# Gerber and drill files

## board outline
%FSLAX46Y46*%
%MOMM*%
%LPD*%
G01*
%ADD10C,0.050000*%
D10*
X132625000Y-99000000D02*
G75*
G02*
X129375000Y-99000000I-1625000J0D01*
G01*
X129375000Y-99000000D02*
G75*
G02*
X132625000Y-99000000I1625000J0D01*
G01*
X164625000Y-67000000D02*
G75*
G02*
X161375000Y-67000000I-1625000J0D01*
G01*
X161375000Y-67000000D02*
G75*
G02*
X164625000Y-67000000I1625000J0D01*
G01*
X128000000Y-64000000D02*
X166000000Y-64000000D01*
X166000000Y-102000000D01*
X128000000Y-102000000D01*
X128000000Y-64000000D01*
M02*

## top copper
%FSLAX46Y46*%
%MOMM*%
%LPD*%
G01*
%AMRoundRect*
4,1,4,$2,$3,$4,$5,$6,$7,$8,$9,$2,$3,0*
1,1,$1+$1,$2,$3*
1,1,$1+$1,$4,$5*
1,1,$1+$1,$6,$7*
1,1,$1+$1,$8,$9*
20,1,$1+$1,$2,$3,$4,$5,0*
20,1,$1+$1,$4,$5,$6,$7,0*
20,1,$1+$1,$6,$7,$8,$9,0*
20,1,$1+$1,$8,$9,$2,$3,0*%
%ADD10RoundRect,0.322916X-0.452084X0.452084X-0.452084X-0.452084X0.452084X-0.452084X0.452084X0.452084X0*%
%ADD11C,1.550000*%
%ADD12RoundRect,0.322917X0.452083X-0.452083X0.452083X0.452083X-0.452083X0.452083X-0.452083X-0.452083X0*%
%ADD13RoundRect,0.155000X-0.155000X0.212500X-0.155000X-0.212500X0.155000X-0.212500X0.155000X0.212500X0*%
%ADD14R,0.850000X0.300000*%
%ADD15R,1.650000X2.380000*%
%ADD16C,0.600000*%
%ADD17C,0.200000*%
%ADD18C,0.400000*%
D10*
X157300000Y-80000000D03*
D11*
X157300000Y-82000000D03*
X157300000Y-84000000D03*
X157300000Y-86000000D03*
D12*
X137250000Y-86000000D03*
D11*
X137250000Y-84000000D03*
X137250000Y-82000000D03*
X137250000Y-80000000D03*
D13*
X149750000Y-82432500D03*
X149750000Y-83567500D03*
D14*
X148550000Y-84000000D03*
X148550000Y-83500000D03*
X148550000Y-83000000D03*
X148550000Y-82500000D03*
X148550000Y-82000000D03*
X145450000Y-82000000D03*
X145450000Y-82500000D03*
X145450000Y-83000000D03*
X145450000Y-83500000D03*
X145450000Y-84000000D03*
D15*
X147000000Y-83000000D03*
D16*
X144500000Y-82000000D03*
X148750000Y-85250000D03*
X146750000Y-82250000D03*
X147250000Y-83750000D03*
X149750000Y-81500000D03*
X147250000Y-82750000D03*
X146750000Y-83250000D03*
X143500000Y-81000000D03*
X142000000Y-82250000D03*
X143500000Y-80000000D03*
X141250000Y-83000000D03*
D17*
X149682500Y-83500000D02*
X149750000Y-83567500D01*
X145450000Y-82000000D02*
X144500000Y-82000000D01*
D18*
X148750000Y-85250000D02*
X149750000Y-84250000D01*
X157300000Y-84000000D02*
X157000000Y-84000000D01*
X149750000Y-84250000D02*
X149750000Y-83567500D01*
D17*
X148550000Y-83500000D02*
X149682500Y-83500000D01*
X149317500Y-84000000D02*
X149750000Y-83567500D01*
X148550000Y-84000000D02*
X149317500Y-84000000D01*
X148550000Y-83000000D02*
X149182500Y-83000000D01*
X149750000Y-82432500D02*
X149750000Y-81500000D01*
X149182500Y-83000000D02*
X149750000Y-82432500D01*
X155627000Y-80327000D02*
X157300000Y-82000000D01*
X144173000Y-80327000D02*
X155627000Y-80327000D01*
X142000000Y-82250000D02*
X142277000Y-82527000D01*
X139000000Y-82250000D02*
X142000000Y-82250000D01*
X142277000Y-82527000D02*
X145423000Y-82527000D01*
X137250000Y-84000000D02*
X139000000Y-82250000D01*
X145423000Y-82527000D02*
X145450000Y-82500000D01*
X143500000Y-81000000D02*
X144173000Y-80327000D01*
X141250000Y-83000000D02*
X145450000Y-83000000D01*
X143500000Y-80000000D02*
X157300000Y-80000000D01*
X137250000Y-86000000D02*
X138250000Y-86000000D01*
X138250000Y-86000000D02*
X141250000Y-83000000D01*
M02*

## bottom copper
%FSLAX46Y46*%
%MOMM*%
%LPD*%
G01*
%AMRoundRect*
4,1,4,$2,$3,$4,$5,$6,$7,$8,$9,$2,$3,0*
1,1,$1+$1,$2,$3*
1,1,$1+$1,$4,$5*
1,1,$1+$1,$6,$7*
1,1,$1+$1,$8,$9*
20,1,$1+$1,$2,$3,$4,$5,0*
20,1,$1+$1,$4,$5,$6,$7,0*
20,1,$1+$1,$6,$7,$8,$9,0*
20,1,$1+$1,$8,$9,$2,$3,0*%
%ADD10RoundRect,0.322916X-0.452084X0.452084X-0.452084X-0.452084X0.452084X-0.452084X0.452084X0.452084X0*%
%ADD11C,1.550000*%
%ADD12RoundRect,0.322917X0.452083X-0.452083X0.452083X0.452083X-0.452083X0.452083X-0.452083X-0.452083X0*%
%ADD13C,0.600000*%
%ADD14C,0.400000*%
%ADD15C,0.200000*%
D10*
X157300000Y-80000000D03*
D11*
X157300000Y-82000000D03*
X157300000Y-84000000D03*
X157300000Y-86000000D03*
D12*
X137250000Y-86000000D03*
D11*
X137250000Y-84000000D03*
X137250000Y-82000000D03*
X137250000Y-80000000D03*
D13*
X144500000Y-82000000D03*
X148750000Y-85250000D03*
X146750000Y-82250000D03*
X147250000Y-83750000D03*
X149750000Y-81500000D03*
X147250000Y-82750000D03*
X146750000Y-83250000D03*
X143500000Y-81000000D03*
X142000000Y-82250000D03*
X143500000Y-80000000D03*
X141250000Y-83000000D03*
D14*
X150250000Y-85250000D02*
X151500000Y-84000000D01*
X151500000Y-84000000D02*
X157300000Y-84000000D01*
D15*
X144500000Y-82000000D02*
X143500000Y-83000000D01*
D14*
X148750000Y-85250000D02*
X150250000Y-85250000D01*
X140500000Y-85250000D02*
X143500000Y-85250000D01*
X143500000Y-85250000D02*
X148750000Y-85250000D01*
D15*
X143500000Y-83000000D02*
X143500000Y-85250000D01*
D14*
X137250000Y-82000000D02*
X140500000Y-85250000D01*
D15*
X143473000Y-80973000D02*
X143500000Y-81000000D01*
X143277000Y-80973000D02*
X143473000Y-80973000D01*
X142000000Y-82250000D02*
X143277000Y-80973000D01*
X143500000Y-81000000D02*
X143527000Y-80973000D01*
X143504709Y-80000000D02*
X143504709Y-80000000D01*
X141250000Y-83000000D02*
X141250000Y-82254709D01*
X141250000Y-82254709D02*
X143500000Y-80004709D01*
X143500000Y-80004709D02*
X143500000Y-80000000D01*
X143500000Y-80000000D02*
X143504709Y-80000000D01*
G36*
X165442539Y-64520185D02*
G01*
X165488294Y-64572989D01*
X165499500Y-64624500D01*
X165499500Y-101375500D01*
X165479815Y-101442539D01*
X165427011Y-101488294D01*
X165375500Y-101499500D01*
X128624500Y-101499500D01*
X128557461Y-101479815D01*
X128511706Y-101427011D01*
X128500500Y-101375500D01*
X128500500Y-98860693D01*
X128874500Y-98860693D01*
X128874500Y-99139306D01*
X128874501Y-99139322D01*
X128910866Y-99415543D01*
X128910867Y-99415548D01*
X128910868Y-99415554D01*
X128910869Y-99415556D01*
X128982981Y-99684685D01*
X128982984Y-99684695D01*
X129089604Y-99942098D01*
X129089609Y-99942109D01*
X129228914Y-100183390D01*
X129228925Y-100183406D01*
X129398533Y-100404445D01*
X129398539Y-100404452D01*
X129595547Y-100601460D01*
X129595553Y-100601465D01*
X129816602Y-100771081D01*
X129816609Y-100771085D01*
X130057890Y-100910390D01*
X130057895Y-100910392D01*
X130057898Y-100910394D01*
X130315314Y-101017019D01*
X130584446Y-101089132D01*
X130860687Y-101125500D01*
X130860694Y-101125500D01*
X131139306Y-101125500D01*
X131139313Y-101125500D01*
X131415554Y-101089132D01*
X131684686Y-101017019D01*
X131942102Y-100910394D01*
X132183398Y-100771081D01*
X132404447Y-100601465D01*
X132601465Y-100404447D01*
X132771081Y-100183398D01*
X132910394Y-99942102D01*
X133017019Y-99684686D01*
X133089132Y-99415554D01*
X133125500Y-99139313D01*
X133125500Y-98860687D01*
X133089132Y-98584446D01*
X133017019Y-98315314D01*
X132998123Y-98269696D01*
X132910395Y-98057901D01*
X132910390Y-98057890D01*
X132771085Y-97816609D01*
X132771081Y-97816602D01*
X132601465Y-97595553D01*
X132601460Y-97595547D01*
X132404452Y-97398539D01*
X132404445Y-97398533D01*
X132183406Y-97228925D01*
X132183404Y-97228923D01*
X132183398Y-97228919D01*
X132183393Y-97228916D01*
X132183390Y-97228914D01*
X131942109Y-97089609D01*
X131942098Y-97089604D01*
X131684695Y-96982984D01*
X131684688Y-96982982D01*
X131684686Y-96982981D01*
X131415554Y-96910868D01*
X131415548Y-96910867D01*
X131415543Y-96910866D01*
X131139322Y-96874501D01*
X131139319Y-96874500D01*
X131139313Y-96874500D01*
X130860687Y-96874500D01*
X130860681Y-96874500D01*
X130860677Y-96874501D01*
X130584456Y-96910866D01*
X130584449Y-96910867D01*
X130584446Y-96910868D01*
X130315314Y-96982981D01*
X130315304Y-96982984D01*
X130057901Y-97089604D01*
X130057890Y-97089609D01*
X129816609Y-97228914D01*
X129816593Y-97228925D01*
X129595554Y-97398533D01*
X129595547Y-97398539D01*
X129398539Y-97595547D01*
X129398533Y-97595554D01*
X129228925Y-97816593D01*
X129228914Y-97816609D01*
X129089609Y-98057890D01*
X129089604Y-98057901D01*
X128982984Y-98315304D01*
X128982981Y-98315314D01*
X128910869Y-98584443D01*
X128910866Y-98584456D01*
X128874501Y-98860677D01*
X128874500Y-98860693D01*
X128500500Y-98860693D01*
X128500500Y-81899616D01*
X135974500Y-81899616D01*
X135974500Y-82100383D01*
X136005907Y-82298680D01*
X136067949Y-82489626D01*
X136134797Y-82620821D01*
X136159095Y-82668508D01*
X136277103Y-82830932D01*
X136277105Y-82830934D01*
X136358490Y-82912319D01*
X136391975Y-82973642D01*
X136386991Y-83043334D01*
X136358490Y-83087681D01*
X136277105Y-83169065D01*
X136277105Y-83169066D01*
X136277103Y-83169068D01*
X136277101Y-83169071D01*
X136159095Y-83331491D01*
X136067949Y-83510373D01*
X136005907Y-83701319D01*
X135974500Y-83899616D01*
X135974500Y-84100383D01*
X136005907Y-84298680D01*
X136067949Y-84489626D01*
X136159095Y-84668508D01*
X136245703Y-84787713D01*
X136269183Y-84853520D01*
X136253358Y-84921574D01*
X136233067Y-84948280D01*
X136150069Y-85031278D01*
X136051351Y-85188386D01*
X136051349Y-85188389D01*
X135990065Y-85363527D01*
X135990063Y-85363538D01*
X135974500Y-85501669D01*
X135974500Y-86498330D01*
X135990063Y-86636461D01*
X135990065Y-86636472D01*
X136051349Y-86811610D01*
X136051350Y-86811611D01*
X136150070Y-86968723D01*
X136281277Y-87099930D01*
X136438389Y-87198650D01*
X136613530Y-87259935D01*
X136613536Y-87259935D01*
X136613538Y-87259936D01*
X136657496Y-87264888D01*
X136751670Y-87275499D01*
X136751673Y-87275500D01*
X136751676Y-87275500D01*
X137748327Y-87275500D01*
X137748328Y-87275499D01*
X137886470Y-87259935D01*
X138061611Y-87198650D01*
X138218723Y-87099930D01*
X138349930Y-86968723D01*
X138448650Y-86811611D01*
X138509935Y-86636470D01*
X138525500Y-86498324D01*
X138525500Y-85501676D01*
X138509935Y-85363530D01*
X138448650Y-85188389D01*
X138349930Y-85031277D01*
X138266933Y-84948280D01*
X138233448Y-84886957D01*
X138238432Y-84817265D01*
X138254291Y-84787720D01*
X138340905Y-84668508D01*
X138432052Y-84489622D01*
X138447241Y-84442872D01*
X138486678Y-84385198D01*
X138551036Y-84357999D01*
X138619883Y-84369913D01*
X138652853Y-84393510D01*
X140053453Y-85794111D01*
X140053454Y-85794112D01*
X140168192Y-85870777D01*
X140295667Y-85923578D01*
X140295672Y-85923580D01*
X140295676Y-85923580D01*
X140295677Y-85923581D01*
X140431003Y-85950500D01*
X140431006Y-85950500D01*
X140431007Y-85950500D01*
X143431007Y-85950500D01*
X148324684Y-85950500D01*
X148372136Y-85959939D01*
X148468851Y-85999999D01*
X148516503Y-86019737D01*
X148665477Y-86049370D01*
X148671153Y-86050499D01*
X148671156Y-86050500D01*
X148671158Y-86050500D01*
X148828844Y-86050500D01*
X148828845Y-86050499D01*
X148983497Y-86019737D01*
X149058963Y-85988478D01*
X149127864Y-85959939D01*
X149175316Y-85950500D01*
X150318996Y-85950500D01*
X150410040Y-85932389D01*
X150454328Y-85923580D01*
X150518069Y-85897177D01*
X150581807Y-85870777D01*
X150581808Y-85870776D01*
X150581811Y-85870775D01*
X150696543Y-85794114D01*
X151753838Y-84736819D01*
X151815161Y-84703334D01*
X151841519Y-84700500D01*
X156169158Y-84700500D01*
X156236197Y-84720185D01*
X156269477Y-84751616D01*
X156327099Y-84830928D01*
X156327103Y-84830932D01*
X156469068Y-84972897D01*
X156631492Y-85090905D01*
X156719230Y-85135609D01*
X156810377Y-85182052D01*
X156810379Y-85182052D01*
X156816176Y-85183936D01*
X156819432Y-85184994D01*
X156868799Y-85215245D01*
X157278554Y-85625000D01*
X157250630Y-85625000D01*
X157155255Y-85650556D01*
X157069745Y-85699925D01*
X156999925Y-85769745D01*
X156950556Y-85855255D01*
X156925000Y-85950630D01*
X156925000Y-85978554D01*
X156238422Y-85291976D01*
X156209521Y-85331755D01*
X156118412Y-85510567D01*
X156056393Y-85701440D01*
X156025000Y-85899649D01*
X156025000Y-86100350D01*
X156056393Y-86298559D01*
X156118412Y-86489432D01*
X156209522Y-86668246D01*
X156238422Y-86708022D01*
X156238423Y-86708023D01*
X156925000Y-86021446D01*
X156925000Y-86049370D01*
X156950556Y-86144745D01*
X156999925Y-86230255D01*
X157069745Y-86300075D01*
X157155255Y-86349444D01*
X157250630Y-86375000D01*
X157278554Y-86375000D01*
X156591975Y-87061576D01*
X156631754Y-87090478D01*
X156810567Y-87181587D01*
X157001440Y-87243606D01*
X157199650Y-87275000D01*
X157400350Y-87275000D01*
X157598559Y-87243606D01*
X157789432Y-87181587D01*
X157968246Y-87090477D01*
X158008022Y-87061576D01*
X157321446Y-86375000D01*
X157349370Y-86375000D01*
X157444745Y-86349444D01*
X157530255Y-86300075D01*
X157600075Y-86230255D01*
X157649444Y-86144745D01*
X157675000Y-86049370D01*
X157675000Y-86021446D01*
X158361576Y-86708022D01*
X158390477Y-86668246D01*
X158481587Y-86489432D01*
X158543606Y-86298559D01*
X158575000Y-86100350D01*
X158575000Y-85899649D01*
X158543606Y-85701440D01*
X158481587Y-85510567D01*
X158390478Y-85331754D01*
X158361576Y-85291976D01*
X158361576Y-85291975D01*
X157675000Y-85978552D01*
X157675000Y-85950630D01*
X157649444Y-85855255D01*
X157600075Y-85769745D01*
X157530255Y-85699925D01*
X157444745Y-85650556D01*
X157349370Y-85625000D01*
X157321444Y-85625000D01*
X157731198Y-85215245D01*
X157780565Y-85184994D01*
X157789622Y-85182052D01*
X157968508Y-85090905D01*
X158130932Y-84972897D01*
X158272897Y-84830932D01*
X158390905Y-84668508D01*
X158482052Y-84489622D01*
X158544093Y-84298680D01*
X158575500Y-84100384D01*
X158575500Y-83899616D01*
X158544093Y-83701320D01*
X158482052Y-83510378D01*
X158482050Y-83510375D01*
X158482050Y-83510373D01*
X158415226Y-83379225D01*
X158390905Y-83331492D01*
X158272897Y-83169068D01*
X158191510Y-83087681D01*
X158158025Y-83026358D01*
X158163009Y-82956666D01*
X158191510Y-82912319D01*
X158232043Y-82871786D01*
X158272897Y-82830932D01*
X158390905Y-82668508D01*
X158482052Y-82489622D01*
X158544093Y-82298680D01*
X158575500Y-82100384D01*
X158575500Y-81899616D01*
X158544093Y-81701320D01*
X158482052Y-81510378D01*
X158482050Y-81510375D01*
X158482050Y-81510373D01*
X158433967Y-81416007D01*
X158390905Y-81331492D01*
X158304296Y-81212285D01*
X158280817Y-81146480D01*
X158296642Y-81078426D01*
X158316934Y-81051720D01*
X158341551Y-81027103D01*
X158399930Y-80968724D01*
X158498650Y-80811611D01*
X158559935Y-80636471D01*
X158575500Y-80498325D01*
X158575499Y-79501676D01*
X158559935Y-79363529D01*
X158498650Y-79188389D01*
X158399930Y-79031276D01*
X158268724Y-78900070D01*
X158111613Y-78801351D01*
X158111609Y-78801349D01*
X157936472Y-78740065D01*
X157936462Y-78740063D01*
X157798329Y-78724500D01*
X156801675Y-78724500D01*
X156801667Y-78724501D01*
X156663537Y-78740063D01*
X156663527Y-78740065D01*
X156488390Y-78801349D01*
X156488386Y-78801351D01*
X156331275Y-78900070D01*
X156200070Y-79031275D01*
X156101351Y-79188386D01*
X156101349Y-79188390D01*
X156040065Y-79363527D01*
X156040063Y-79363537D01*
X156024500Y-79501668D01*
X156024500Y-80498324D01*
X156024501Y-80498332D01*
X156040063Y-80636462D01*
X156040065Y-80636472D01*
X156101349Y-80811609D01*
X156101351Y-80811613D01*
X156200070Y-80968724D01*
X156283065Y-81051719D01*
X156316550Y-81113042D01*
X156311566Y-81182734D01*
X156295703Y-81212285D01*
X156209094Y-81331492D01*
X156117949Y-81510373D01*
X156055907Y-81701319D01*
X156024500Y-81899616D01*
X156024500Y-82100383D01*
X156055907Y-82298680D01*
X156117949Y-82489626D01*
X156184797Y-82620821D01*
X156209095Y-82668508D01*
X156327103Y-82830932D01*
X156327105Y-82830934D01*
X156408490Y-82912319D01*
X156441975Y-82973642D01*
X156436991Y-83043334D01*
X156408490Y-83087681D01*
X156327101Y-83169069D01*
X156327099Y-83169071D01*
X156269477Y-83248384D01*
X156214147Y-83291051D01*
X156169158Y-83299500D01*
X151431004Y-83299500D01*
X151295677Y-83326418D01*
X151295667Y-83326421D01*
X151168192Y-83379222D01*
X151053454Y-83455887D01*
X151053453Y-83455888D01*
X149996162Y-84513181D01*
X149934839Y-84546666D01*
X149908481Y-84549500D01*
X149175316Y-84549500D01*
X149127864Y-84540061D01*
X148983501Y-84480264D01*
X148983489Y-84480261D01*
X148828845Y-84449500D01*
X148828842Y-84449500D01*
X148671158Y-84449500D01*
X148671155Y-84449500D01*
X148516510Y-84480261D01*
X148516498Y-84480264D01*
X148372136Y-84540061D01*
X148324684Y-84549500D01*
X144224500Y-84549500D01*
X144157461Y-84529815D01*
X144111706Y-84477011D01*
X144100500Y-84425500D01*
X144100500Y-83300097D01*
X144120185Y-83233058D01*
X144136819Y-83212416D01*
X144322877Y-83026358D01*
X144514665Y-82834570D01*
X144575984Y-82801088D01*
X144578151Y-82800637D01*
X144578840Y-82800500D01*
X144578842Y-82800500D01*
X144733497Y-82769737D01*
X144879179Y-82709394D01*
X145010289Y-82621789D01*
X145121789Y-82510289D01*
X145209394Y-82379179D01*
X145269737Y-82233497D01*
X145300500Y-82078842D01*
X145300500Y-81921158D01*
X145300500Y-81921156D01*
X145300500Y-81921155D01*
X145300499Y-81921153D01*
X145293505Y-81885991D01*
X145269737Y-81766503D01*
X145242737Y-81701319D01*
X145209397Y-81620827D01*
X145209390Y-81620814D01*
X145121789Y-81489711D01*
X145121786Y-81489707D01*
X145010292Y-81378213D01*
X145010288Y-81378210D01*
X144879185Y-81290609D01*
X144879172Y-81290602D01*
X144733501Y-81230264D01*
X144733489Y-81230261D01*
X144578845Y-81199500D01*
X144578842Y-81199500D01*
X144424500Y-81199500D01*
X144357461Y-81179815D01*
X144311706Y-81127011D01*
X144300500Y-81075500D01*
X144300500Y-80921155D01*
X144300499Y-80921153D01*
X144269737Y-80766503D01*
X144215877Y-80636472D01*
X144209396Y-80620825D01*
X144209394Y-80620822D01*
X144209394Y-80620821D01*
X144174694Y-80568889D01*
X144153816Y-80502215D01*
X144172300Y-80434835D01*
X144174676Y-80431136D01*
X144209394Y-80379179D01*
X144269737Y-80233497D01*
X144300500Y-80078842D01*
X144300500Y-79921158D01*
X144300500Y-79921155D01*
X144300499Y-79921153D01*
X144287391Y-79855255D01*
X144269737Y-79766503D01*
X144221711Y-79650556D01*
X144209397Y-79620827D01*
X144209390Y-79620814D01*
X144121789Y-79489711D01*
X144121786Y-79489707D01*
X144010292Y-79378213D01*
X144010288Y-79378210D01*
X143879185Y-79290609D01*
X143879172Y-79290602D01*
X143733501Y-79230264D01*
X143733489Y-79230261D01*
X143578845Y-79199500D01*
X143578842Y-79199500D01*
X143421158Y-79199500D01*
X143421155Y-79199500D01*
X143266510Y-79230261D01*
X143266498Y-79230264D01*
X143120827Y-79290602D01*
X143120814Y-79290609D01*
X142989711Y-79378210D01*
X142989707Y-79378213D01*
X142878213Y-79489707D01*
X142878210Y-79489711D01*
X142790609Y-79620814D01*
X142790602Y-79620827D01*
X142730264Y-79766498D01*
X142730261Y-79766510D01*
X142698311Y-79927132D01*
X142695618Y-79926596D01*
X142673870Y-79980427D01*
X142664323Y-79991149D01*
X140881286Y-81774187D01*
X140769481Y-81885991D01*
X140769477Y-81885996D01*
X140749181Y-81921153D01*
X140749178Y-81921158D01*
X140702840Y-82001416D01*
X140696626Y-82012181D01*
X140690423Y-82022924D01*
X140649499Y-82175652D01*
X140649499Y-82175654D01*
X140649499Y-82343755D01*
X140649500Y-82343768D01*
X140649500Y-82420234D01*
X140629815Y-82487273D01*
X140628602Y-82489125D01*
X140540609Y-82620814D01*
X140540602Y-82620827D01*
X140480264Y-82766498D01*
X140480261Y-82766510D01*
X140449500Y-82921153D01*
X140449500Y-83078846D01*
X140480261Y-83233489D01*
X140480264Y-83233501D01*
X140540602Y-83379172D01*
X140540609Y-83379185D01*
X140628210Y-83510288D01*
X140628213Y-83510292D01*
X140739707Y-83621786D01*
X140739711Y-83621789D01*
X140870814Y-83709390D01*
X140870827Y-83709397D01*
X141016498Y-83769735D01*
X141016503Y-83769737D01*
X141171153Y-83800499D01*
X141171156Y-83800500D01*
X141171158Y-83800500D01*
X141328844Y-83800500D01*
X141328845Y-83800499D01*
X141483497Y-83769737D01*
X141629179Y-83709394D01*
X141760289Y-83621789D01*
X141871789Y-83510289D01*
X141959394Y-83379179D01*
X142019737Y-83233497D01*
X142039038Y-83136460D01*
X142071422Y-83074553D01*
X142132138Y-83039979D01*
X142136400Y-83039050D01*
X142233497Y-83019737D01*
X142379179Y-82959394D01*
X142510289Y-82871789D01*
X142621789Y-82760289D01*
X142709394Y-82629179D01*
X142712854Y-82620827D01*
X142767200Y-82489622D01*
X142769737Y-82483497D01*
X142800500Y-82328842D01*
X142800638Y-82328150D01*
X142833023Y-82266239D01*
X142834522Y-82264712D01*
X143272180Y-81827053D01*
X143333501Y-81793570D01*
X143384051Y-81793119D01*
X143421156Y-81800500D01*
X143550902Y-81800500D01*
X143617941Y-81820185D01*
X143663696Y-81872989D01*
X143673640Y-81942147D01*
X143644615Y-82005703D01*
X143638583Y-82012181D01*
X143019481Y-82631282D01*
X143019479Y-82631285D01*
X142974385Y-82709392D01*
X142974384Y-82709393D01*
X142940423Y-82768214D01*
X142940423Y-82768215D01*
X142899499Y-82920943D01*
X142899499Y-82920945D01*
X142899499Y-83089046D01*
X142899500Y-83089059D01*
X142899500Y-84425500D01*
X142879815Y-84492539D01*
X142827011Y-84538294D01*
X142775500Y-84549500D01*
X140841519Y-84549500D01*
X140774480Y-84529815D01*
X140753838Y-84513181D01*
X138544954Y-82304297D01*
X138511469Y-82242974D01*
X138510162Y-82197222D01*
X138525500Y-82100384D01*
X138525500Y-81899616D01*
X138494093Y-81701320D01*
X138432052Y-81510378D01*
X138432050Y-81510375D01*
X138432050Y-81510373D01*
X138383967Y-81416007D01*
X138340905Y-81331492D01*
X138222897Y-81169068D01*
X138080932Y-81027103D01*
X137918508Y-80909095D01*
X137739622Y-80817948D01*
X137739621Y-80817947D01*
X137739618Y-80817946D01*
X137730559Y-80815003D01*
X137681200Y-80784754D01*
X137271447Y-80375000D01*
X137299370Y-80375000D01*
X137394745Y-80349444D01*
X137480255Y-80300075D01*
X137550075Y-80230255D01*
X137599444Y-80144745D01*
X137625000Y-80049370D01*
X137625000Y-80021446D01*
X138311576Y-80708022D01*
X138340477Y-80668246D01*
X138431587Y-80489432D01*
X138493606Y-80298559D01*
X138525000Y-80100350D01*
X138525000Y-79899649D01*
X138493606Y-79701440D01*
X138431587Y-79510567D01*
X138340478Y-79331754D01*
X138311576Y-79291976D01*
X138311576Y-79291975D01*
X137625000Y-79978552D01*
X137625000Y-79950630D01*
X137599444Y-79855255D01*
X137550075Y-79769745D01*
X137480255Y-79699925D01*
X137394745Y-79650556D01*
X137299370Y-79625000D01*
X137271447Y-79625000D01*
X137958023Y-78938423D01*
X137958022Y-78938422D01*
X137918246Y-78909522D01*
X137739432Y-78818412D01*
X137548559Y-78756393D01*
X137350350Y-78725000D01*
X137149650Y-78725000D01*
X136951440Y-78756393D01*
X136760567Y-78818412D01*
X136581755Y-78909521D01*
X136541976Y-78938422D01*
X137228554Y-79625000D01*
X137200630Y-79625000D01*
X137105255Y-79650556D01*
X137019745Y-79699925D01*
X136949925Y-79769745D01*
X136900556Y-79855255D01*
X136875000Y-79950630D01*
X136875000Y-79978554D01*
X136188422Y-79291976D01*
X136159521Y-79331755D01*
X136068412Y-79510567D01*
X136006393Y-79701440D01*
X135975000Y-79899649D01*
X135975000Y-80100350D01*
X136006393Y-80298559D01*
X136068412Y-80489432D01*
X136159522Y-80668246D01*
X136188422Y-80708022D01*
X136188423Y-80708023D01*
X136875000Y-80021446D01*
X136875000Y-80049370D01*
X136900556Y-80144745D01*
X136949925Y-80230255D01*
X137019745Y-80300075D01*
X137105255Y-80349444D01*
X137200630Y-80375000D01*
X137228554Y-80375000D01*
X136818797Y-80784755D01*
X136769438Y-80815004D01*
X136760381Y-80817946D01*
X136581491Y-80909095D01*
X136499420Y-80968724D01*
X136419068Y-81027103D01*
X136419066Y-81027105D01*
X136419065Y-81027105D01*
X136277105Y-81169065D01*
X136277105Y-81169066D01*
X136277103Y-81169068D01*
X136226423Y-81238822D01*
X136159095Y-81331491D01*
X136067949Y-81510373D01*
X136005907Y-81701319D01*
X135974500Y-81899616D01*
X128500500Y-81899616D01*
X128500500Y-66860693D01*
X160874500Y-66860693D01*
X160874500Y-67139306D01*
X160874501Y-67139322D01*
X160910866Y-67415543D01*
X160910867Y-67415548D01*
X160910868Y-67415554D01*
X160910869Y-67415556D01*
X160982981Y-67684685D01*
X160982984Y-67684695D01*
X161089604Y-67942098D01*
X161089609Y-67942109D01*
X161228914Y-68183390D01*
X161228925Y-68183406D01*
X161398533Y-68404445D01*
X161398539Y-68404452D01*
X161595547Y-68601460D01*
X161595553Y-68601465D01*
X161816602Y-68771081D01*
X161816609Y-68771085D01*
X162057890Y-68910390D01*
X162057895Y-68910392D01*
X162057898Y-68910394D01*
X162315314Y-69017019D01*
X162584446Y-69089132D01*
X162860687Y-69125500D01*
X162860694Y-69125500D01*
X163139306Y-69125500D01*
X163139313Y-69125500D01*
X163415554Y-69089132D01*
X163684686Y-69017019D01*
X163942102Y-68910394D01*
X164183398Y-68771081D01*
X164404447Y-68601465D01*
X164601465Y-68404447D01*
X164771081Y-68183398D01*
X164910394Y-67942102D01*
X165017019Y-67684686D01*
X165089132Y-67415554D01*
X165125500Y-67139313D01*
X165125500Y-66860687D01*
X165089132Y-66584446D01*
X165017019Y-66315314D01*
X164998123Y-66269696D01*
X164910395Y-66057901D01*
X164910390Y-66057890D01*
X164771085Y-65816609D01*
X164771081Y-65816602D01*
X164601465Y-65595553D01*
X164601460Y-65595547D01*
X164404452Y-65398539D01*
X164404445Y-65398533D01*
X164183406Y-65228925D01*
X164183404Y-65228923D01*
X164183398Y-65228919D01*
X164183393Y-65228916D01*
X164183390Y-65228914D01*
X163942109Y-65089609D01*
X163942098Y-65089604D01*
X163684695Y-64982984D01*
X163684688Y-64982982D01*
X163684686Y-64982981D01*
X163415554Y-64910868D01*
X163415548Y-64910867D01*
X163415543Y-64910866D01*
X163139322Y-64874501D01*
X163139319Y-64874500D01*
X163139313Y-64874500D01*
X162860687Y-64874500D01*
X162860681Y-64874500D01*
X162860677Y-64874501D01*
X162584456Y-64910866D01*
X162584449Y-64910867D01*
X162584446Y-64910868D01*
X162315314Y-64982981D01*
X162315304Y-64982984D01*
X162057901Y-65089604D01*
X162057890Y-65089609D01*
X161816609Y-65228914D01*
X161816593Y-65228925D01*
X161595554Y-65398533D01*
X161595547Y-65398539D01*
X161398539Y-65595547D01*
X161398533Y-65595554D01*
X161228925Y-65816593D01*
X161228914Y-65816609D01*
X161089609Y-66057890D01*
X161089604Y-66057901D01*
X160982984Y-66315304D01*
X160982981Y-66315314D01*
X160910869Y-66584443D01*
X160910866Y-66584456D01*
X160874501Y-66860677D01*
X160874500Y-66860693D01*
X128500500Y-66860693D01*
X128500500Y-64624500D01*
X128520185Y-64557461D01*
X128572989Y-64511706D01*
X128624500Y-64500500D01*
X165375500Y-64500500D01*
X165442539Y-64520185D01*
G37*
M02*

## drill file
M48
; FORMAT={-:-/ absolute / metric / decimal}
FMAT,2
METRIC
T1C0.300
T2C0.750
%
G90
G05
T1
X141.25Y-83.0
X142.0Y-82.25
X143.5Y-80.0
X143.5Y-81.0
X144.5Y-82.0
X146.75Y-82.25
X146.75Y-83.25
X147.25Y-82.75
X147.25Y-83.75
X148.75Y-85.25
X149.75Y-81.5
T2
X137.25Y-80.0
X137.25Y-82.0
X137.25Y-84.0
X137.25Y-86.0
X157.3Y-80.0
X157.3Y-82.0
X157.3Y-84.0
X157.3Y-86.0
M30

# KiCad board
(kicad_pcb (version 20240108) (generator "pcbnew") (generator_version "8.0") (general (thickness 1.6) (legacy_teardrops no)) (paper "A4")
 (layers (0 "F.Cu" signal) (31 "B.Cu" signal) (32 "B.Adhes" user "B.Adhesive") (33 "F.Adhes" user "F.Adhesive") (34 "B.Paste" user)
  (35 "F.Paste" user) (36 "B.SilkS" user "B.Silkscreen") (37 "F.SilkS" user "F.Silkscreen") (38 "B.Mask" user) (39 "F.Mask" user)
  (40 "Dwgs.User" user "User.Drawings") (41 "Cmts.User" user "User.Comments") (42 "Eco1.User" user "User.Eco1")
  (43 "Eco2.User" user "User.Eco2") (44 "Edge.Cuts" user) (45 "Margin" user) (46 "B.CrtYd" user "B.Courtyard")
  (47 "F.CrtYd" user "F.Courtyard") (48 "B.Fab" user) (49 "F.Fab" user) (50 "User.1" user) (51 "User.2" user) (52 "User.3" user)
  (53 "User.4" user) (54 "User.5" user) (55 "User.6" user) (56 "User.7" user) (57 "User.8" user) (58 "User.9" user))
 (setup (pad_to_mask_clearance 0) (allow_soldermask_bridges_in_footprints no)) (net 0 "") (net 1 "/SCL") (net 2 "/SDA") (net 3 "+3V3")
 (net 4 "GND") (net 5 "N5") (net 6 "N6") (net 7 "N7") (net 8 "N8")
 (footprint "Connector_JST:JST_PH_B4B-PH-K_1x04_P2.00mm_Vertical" (layer "F.Cu") (at 157.3 80 -90)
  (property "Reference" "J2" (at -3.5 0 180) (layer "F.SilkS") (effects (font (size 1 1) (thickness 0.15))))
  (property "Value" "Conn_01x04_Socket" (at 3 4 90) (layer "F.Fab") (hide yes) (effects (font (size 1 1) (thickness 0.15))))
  (pad "1" thru_hole roundrect (at 0 0 270) (size 1.55 1.55) (drill 0.75) (layers "*.Cu" "*.Mask") (remove_unused_layers no)
   (roundrect_rratio 0.208333) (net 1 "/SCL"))
  (pad "2" thru_hole circle (at 2 0 270) (size 1.55 1.55) (drill 0.75) (layers "*.Cu" "*.Mask") (remove_unused_layers no) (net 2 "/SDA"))
  (pad "3" thru_hole circle (at 4 0 270) (size 1.55 1.55) (drill 0.75) (layers "*.Cu" "*.Mask") (remove_unused_layers no) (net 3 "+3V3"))
  (pad "4" thru_hole circle (at 6 0 270) (size 1.55 1.55) (drill 0.75) (layers "*.Cu" "*.Mask") (remove_unused_layers no) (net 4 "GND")))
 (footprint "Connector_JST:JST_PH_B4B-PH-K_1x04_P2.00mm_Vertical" (layer "F.Cu") (at 137.25 86 90)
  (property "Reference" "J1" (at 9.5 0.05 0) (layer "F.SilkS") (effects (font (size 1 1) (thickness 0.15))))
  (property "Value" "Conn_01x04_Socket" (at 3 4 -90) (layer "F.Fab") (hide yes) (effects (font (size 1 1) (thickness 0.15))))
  (pad "1" thru_hole roundrect (at 0 0 90) (size 1.55 1.55) (drill 0.75) (layers "*.Cu" "*.Mask") (remove_unused_layers no)
   (roundrect_rratio 0.2083333333) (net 1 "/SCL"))
  (pad "2" thru_hole circle (at 2 0 90) (size 1.55 1.55) (drill 0.75) (layers "*.Cu" "*.Mask") (remove_unused_layers no) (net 2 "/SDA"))
  (pad "3" thru_hole circle (at 4 0 90) (size 1.55 1.55) (drill 0.75) (layers "*.Cu" "*.Mask") (remove_unused_layers no) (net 3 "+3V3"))
  (pad "4" thru_hole circle (at 6 0 90) (size 1.55 1.55) (drill 0.75) (layers "*.Cu" "*.Mask") (remove_unused_layers no) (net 4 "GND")))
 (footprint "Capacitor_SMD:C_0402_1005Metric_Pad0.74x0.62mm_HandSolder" (layer "F.Cu") (at 149.75 83 -90)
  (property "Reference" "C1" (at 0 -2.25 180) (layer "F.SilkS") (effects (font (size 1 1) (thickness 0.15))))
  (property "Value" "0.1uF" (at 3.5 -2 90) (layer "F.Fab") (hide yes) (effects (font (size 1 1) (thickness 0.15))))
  (pad "1" smd roundrect (at -0.5675 0 270) (size 0.735 0.62) (layers "F.Cu" "F.Paste" "F.Mask") (roundrect_rratio 0.25) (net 4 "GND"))
  (pad "2" smd roundrect (at 0.5675 0 270) (size 0.735 0.62) (layers "F.Cu" "F.Paste" "F.Mask") (roundrect_rratio 0.25) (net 3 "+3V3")))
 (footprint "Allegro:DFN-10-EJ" (layer "F.Cu") (at 147 83 90)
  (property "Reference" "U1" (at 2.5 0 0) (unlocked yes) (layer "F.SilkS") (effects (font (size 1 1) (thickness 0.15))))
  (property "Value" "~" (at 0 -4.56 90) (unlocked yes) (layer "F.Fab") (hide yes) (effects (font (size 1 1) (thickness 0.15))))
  (pad "1" smd rect (at -1 1.55 90) (size 0.3 0.85) (layers "F.Cu" "F.Paste" "F.Mask") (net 3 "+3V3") (thermal_bridge_angle 45))
  (pad "2" smd rect (at -0.5 1.55 90) (size 0.3 0.85) (layers "F.Cu" "F.Paste" "F.Mask") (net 3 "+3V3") (thermal_bridge_angle 45))
  (pad "3" smd rect (at 0 1.55 90) (size 0.3 0.85) (layers "F.Cu" "F.Paste" "F.Mask") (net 4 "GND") (thermal_bridge_angle 45))
  (pad "4" smd rect (at 0.5 1.55 90) (size 0.3 0.85) (layers "F.Cu" "F.Paste" "F.Mask") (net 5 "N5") (thermal_bridge_angle 45))
  (pad "5" smd rect (at 1 1.55 90) (size 0.3 0.85) (layers "F.Cu" "F.Paste" "F.Mask") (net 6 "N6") (thermal_bridge_angle 45))
  (pad "6" smd rect (at 1 -1.55 90) (size 0.3 0.85) (layers "F.Cu" "F.Paste" "F.Mask") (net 3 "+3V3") (thermal_bridge_angle 45))
  (pad "7" smd rect (at 0.5 -1.55 90) (size 0.3 0.85) (layers "F.Cu" "F.Paste" "F.Mask") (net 2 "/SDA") (thermal_bridge_angle 45))
  (pad "8" smd rect (at 0 -1.55 90) (size 0.3 0.85) (layers "F.Cu" "F.Paste" "F.Mask") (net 1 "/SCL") (thermal_bridge_angle 45))
  (pad "9" smd rect (at -0.5 -1.55 90) (size 0.3 0.85) (layers "F.Cu" "F.Paste" "F.Mask") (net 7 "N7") (thermal_bridge_angle 45))
  (pad "10" smd rect (at -1 -1.55 90) (size 0.3 0.85) (layers "F.Cu" "F.Paste" "F.Mask") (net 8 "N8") (thermal_bridge_angle 45))
  (pad "11" smd rect (at 0 0 90) (size 2.38 1.65) (layers "F.Cu" "F.Paste" "F.Mask") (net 4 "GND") (thermal_bridge_angle 45)))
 (gr_circle (center 131 99) (end 132.625 99) (stroke (width 0.05) (type default)) (fill none) (layer "Edge.Cuts"))
 (gr_circle (center 163 67) (end 164.625 67) (stroke (width 0.05) (type default)) (fill none) (layer "Edge.Cuts"))
 (gr_rect (start 128 64) (end 166 102) (stroke (width 0.05) (type default)) (fill none) (layer "Edge.Cuts"))
 (segment (start 149.6825 83.5) (end 149.75 83.5675) (width 0.2) (layer "F.Cu") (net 3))
 (segment (start 145.45 82) (end 144.5 82) (width 0.2) (layer "F.Cu") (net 3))
 (segment (start 148.75 85.25) (end 149.75 84.25) (width 0.4) (layer "F.Cu") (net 3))
 (segment (start 157.3 84) (end 157 84) (width 0.4) (layer "F.Cu") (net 3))
 (segment (start 149.75 84.25) (end 149.75 83.5675) (width 0.4) (layer "F.Cu") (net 3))
 (segment (start 148.55 83.5) (end 149.6825 83.5) (width 0.2) (layer "F.Cu") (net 3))
 (segment (start 149.3175 84) (end 149.75 83.5675) (width 0.2) (layer "F.Cu") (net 3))
 (segment (start 148.55 84) (end 149.3175 84) (width 0.2) (layer "F.Cu") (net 3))
 (via (at 144.5 82) (size 0.6) (drill 0.3) (layers "F.Cu" "B.Cu") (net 3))
 (via (at 148.75 85.25) (size 0.6) (drill 0.3) (layers "F.Cu" "B.Cu") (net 3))
 (segment (start 150.25 85.25) (end 151.5 84) (width 0.4) (layer "B.Cu") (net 3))
 (segment (start 151.5 84) (end 157.3 84) (width 0.4) (layer "B.Cu") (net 3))
 (segment (start 144.5 82) (end 143.5 83) (width 0.2) (layer "B.Cu") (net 3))
 (segment (start 148.75 85.25) (end 150.25 85.25) (width 0.4) (layer "B.Cu") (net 3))
 (segment (start 140.5 85.25) (end 143.5 85.25) (width 0.4) (layer "B.Cu") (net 3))
 (segment (start 143.5 85.25) (end 148.75 85.25) (width 0.4) (layer "B.Cu") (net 3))
 (segment (start 143.5 83) (end 143.5 85.25) (width 0.2) (layer "B.Cu") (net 3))
 (segment (start 137.25 82) (end 140.5 85.25) (width 0.4) (layer "B.Cu") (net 3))
 (segment (start 148.55 83) (end 149.1825 83) (width 0.2) (layer "F.Cu") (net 4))
 (segment (start 149.75 82.4325) (end 149.75 81.5) (width 0.2) (layer "F.Cu") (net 4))
 (segment (start 149.1825 83) (end 149.75 82.4325) (width 0.2) (layer "F.Cu") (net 4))
 (via (at 146.75 82.25) (size 0.6) (drill 0.3) (layers "F.Cu" "B.Cu") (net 4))
 (via (at 147.25 83.75) (size 0.6) (drill 0.3) (layers "F.Cu" "B.Cu") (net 4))
 (via (at 149.75 81.5) (size 0.6) (drill 0.3) (layers "F.Cu" "B.Cu") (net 4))
 (via (at 147.25 82.75) (size 0.6) (drill 0.3) (layers "F.Cu" "B.Cu") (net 4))
 (via (at 146.75 83.25) (size 0.6) (drill 0.3) (layers "F.Cu" "B.Cu") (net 4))
 (segment (start 155.627 80.327) (end 157.3 82) (width 0.2) (layer "F.Cu") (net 2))
 (segment (start 144.173 80.327) (end 155.627 80.327) (width 0.2) (layer "F.Cu") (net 2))
 (segment (start 142 82.25) (end 142.277 82.527) (width 0.2) (layer "F.Cu") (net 2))
 (segment (start 139 82.25) (end 142 82.25) (width 0.2) (layer "F.Cu") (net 2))
 (segment (start 142.277 82.527) (end 145.423 82.527) (width 0.2) (layer "F.Cu") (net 2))
 (segment (start 137.25 84) (end 139 82.25) (width 0.2) (layer "F.Cu") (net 2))
 (segment (start 145.423 82.527) (end 145.45 82.5) (width 0.2) (layer "F.Cu") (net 2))
 (segment (start 143.5 81) (end 144.173 80.327) (width 0.2) (layer "F.Cu") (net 2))
 (via (at 143.5 81) (size 0.6) (drill 0.3) (layers "F.Cu" "B.Cu") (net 2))
 (via (at 142 82.25) (size 0.6) (drill 0.3) (layers "F.Cu" "B.Cu") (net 2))
 (segment (start 143.473 80.973) (end 143.5 81) (width 0.2) (layer "B.Cu") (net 2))
 (segment (start 143.277 80.973) (end 143.473 80.973) (width 0.2) (layer "B.Cu") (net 2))
 (segment (start 142 82.25) (end 143.277 80.973) (width 0.2) (layer "B.Cu") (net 2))
 (segment (start 143.5 81) (end 143.527 80.973) (width 0.2) (layer "B.Cu") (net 2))
 (segment (start 141.25 83) (end 145.45 83) (width 0.2) (layer "F.Cu") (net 1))
 (segment (start 143.5 80) (end 157.3 80) (width 0.2) (layer "F.Cu") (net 1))
 (segment (start 137.25 86) (end 138.25 86) (width 0.2) (layer "F.Cu") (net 1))
 (segment (start 138.25 86) (end 141.25 83) (width 0.2) (layer "F.Cu") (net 1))
 (via (at 143.5 80) (size 0.6) (drill 0.3) (layers "F.Cu" "B.Cu") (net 1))
 (via (at 141.25 83) (size 0.6) (drill 0.3) (layers "F.Cu" "B.Cu") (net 1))
 (segment (start 143.504709 80) (end 143.504709 80) (width 0.2) (layer "B.Cu") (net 1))
 (segment (start 141.25 83) (end 141.25 82.254709) (width 0.2) (layer "B.Cu") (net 1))
 (segment (start 141.25 82.254709) (end 143.5 80.004709) (width 0.2) (layer "B.Cu") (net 1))
 (segment (start 143.5 80.004709) (end 143.5 80) (width 0.2) (layer "B.Cu") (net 1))
 (segment (start 143.5 80) (end 143.504709 80) (width 0.2) (layer "B.Cu") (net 1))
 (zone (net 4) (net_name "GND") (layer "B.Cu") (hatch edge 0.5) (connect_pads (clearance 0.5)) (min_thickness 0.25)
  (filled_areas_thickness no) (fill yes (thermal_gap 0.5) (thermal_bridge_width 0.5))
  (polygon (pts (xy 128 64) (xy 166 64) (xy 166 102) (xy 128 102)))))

